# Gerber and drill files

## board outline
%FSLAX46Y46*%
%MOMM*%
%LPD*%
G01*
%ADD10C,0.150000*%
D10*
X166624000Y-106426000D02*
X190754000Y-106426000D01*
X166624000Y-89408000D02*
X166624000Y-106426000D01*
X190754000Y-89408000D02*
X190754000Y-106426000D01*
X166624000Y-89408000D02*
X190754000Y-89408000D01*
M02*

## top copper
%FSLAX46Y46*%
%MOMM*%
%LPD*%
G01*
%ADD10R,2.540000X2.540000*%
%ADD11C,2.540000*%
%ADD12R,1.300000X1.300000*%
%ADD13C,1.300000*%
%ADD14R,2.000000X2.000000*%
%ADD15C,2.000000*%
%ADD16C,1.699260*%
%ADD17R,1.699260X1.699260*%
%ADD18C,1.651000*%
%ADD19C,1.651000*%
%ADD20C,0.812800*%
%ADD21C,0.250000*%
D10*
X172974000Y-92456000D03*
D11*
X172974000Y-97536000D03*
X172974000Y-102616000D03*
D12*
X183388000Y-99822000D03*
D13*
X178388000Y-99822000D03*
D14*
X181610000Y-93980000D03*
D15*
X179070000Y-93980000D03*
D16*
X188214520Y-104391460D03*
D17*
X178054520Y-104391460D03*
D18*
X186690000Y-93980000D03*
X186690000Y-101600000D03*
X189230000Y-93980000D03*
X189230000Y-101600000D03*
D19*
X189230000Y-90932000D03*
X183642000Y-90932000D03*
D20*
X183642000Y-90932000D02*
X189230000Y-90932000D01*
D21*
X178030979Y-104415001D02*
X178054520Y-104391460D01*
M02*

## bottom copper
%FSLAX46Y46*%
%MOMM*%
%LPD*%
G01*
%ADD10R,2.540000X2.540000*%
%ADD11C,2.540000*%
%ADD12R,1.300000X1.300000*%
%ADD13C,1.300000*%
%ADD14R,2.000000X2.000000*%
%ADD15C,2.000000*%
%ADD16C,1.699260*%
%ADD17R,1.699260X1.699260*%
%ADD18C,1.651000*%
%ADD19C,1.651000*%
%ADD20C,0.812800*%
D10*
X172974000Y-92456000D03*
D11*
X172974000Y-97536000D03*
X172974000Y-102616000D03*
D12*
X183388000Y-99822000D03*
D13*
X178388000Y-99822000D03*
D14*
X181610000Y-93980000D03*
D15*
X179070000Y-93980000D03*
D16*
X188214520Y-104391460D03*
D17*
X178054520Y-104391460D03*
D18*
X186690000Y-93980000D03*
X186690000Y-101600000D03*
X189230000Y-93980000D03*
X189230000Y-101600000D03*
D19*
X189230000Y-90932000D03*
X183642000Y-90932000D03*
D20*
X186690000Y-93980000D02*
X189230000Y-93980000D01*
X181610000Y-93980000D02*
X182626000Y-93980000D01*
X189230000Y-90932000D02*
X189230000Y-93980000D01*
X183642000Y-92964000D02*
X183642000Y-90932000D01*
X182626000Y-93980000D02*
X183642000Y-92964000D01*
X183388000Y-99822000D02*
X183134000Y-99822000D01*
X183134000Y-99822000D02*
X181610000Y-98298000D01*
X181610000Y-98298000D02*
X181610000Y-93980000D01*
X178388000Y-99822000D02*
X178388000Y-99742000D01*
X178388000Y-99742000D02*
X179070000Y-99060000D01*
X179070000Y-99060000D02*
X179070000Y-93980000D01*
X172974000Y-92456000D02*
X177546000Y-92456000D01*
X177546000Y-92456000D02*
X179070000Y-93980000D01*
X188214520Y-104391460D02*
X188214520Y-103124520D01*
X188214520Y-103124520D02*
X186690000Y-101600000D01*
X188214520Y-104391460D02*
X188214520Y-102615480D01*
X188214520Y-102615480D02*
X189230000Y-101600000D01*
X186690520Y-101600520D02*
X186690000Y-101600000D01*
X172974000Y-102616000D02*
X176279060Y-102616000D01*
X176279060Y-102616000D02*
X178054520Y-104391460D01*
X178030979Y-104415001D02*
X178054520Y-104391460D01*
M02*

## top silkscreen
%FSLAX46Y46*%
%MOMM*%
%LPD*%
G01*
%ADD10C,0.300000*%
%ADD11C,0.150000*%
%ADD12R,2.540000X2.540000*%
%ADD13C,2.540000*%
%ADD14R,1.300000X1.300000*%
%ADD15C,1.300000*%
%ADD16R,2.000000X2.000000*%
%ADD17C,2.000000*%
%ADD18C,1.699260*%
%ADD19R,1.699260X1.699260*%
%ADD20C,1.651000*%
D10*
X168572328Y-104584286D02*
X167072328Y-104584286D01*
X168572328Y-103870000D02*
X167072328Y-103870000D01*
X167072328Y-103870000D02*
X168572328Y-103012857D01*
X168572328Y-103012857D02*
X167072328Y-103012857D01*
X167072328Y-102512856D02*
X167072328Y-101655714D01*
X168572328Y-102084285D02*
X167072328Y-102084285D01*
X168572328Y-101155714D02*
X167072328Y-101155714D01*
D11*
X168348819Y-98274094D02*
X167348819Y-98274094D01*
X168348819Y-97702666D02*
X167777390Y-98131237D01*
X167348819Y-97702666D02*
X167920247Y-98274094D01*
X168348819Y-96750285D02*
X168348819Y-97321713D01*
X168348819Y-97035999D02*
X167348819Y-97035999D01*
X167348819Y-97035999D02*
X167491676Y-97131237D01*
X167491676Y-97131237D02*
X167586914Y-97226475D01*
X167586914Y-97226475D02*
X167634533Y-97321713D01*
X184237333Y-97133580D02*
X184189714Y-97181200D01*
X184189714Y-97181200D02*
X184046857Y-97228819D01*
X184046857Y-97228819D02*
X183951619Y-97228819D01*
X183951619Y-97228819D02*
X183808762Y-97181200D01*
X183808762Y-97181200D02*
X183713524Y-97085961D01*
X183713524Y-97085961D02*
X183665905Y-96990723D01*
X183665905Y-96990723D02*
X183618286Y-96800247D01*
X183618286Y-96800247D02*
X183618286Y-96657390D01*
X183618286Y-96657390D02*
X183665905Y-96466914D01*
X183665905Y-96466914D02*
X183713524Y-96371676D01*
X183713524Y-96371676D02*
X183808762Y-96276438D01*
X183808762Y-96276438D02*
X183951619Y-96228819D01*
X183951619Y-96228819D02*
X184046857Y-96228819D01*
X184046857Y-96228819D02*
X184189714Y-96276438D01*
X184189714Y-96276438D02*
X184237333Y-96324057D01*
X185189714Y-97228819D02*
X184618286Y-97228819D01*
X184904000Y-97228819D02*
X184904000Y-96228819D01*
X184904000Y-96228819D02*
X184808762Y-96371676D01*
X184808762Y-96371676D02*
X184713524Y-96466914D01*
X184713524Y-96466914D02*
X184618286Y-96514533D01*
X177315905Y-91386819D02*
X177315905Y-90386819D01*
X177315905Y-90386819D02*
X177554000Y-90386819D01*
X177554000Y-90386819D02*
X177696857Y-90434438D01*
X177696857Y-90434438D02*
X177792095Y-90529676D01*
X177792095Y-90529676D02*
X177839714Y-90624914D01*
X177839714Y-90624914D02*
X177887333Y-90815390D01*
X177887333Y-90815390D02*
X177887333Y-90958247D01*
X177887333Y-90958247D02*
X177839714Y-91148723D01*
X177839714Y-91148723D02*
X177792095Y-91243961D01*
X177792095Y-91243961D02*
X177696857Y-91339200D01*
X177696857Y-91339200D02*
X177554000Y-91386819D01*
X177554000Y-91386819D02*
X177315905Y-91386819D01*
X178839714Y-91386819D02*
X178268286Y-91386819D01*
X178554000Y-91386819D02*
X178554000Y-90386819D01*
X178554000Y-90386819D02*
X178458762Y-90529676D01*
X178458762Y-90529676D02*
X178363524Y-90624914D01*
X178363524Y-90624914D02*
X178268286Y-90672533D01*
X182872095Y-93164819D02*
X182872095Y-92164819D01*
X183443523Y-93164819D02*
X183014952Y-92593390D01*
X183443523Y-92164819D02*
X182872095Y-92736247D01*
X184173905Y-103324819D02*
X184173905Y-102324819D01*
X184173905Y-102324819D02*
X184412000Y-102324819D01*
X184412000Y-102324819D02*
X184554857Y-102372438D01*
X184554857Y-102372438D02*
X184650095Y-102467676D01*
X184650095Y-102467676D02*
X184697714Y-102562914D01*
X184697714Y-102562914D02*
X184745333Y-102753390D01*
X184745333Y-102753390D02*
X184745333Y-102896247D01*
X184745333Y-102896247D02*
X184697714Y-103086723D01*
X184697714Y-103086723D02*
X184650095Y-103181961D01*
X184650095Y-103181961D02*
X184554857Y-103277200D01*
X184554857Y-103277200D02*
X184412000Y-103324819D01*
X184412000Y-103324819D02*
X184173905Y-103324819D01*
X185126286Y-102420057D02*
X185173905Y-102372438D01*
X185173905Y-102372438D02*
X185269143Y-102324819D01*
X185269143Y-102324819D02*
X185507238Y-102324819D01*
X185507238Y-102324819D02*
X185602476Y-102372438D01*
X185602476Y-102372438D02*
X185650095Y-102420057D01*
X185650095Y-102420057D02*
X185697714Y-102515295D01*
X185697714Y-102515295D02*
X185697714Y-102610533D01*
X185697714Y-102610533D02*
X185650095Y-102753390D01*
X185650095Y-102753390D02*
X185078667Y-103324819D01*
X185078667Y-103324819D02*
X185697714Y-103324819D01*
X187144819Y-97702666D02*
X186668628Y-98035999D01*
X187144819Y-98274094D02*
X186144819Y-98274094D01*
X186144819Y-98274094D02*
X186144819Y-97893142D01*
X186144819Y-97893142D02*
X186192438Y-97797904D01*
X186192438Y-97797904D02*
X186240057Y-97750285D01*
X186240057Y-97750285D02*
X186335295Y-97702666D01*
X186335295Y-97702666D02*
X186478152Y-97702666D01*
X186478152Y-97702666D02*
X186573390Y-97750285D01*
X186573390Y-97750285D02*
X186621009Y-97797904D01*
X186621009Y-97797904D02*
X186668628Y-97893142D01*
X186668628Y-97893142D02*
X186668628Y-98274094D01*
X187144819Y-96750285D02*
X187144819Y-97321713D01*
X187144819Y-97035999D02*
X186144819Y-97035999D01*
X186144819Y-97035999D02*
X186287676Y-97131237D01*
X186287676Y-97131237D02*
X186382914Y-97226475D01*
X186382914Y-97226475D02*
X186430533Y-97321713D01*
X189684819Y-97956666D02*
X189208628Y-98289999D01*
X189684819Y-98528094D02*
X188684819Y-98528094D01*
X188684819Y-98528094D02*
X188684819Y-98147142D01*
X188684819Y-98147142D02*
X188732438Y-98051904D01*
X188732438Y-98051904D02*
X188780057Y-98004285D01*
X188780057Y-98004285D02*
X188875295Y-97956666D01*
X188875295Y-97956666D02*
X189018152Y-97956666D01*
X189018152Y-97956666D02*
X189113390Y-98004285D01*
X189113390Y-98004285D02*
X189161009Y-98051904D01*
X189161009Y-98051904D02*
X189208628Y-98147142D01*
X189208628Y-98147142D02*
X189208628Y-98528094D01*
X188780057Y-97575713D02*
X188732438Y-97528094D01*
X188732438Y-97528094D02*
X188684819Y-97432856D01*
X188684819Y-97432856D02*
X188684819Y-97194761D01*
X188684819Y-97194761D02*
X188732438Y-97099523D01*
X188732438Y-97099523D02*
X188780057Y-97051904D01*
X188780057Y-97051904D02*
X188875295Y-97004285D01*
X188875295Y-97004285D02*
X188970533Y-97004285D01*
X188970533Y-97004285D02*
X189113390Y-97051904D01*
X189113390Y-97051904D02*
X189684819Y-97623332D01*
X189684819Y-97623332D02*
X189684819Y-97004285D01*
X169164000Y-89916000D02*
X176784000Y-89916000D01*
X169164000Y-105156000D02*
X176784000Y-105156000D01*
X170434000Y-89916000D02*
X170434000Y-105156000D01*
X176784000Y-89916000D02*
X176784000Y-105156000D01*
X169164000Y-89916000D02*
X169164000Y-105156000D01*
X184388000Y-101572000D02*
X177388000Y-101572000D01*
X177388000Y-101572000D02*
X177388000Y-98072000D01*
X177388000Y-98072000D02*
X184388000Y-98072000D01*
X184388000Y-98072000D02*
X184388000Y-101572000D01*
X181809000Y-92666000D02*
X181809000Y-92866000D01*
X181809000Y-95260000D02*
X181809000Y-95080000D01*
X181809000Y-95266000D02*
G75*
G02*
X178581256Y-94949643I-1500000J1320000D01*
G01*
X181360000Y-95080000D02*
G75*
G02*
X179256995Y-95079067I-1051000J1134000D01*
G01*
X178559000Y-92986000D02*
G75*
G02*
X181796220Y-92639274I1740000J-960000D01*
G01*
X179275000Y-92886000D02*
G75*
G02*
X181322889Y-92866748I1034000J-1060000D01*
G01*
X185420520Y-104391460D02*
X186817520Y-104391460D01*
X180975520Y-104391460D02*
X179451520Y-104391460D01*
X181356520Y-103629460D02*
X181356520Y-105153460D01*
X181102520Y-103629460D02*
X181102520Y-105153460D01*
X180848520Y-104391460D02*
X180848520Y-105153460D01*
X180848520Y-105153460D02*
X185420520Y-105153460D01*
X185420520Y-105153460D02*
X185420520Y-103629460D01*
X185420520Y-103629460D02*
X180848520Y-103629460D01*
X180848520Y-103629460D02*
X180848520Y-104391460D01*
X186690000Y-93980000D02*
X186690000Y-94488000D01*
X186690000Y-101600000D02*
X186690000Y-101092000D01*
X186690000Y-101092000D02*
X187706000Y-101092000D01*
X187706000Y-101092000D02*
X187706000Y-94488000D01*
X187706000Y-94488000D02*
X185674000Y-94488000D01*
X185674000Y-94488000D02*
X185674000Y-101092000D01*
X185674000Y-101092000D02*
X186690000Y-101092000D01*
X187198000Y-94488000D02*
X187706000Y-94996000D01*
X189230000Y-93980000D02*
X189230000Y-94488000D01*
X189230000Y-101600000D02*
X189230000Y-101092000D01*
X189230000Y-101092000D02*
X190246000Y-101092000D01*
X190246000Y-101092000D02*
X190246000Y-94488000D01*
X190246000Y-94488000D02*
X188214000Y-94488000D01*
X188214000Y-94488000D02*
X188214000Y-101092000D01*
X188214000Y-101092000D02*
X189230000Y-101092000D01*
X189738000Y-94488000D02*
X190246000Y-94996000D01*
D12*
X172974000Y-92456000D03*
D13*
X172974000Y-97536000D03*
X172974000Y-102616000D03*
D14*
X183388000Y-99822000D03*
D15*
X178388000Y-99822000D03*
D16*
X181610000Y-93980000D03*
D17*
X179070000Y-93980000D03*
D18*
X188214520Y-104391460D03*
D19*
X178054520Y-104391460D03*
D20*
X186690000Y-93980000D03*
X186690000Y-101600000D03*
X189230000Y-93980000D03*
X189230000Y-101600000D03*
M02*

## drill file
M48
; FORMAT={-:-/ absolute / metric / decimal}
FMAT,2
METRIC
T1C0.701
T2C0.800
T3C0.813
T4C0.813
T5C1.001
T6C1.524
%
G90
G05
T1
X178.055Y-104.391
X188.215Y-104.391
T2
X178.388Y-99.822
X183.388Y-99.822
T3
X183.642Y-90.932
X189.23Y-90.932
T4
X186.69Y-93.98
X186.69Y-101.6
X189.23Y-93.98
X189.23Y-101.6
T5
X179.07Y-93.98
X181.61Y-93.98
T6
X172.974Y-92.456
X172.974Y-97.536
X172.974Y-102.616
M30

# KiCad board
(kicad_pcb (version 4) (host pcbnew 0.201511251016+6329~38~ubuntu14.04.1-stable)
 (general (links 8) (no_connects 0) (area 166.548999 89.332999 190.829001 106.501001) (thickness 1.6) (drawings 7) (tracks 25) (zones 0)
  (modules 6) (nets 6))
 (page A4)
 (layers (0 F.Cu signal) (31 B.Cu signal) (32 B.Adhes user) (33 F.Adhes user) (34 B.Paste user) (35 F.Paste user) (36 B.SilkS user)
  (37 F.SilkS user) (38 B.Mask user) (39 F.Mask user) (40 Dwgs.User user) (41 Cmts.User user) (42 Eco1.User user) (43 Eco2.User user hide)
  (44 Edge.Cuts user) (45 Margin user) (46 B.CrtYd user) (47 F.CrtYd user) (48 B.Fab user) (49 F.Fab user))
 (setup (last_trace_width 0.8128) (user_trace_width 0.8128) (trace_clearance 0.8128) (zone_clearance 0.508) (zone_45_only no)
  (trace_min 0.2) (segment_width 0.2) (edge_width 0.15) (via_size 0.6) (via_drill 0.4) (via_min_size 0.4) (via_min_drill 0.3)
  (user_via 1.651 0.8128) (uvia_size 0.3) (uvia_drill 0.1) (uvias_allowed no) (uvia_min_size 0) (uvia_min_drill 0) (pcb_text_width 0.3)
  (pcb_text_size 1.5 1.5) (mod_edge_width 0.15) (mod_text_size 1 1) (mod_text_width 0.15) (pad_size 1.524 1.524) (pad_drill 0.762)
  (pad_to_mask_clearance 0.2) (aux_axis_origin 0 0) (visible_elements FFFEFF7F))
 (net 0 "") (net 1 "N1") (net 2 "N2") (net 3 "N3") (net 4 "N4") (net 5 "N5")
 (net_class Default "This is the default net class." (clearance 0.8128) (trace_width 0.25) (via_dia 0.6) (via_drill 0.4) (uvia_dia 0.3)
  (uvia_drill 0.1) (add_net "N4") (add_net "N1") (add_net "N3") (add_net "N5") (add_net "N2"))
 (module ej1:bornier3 (layer F.Cu) (at 172.974 97.536 270)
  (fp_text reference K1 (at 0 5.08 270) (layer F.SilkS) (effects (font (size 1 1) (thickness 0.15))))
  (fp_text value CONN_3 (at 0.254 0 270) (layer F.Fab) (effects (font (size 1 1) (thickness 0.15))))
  (fp_line (start -7.62 3.81) (end -7.62 -3.81) (layer F.SilkS) (width 0.15))
  (fp_line (start 7.62 3.81) (end 7.62 -3.81) (layer F.SilkS) (width 0.15))
  (fp_line (start -7.62 2.54) (end 7.62 2.54) (layer F.SilkS) (width 0.15))
  (fp_line (start -7.62 -3.81) (end 7.62 -3.81) (layer F.SilkS) (width 0.15))
  (fp_line (start -7.62 3.81) (end 7.62 3.81) (layer F.SilkS) (width 0.15))
  (pad 1 thru_hole rect (at -5.08 0 270) (size 2.54 2.54) (drill 1.524) (layers *.Cu *.Mask F.SilkS) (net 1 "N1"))
  (pad 2 thru_hole circle (at 0 0 270) (size 2.54 2.54) (drill 1.524) (layers *.Cu *.Mask F.SilkS) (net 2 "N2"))
  (pad 3 thru_hole circle (at 5.08 0 270) (size 2.54 2.54) (drill 1.524) (layers *.Cu *.Mask F.SilkS) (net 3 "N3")))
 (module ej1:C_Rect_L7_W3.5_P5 (layer F.Cu) (at 183.388 99.822 180)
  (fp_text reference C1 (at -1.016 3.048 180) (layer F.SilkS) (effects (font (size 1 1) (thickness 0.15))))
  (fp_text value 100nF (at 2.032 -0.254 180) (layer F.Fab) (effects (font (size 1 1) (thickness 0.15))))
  (fp_line (start -1 -1.75) (end 6 -1.75) (layer F.SilkS) (width 0.15))
  (fp_line (start 6 -1.75) (end 6 1.75) (layer F.SilkS) (width 0.15))
  (fp_line (start 6 1.75) (end -1 1.75) (layer F.SilkS) (width 0.15))
  (fp_line (start -1 1.75) (end -1 -1.75) (layer F.SilkS) (width 0.15))
  (pad 1 thru_hole rect (at 0 0 180) (size 1.3 1.3) (drill 0.8) (layers *.Cu *.Mask F.SilkS) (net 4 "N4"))
  (pad 2 thru_hole circle (at 5 0 180) (size 1.3 1.3) (drill 0.8) (layers *.Cu *.Mask F.SilkS) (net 1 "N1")))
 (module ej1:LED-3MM (layer F.Cu) (at 181.61 93.98 180)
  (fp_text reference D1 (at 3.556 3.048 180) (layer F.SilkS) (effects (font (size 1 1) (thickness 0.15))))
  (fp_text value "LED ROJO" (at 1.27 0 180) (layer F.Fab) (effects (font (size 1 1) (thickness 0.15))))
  (fp_line (start -0.199 1.314) (end -0.199 1.114) (layer F.SilkS) (width 0.15))
  (fp_line (start -0.199 -1.28) (end -0.199 -1.1) (layer F.SilkS) (width 0.15))
  (fp_arc (start 1.301 0.034) (end -0.199 -1.286) (angle 108.5) (layer F.SilkS) (width 0.15))
  (fp_arc (start 1.301 0.034) (end 0.25 -1.1) (angle 85.7) (layer F.SilkS) (width 0.15))
  (fp_arc (start 1.311 0.034) (end 3.051 0.994) (angle 110) (layer F.SilkS) (width 0.15))
  (fp_arc (start 1.301 0.034) (end 2.335 1.094) (angle 87.5) (layer F.SilkS) (width 0.15))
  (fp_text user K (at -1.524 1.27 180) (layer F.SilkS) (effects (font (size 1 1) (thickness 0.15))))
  (pad 1 thru_hole rect (at 0 0 270) (size 2 2) (drill 1.00076) (layers *.Cu *.Mask F.SilkS) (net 4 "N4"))
  (pad 2 thru_hole circle (at 2.54 0 180) (size 2 2) (drill 1.00076) (layers *.Cu *.Mask F.SilkS) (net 1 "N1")))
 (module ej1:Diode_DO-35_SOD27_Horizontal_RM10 (layer F.Cu) (at 178.054 104.394)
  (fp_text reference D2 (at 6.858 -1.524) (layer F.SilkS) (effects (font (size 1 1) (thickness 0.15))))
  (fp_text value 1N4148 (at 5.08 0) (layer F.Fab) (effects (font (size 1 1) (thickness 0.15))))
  (fp_line (start 7.36652 -0.00254) (end 8.76352 -0.00254) (layer F.SilkS) (width 0.15))
  (fp_line (start 2.92152 -0.00254) (end 1.39752 -0.00254) (layer F.SilkS) (width 0.15))
  (fp_line (start 3.30252 -0.76454) (end 3.30252 0.75946) (layer F.SilkS) (width 0.15))
  (fp_line (start 3.04852 -0.76454) (end 3.04852 0.75946) (layer F.SilkS) (width 0.15))
  (fp_line (start 2.79452 -0.00254) (end 2.79452 0.75946) (layer F.SilkS) (width 0.15))
  (fp_line (start 2.79452 0.75946) (end 7.36652 0.75946) (layer F.SilkS) (width 0.15))
  (fp_line (start 7.36652 0.75946) (end 7.36652 -0.76454) (layer F.SilkS) (width 0.15))
  (fp_line (start 7.36652 -0.76454) (end 2.79452 -0.76454) (layer F.SilkS) (width 0.15))
  (fp_line (start 2.79452 -0.76454) (end 2.79452 -0.00254) (layer F.SilkS) (width 0.15))
  (pad 2 thru_hole circle (at 10.16052 -0.00254 180) (size 1.69926 1.69926) (drill 0.70104) (layers *.Cu *.Mask F.SilkS) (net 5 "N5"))
  (pad 1 thru_hole rect (at 0.00052 -0.00254 180) (size 1.69926 1.69926) (drill 0.70104) (layers *.Cu *.Mask F.SilkS) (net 3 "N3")))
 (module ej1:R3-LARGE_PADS (layer F.Cu) (at 186.69 97.79 270)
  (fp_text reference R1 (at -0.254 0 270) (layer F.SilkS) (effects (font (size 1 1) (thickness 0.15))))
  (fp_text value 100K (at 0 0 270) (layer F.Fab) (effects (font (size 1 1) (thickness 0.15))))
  (fp_line (start -3.81 0) (end -3.302 0) (layer F.SilkS) (width 0.15))
  (fp_line (start 3.81 0) (end 3.302 0) (layer F.SilkS) (width 0.15))
  (fp_line (start 3.302 0) (end 3.302 -1.016) (layer F.SilkS) (width 0.15))
  (fp_line (start 3.302 -1.016) (end -3.302 -1.016) (layer F.SilkS) (width 0.15))
  (fp_line (start -3.302 -1.016) (end -3.302 1.016) (layer F.SilkS) (width 0.15))
  (fp_line (start -3.302 1.016) (end 3.302 1.016) (layer F.SilkS) (width 0.15))
  (fp_line (start 3.302 1.016) (end 3.302 0) (layer F.SilkS) (width 0.15))
  (fp_line (start -3.302 -0.508) (end -2.794 -1.016) (layer F.SilkS) (width 0.15))
  (pad 1 thru_hole circle (at -3.81 0 270) (size 1.651 1.651) (drill 0.8128) (layers *.Cu *.Mask F.SilkS) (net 4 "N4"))
  (pad 2 thru_hole circle (at 3.81 0 270) (size 1.651 1.651) (drill 0.8128) (layers *.Cu *.Mask F.SilkS) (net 5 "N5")))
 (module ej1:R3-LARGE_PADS (layer F.Cu) (at 189.23 97.79 270)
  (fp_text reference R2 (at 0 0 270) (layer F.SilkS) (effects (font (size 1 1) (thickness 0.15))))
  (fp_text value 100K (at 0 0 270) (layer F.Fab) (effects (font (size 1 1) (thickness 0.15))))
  (fp_line (start -3.81 0) (end -3.302 0) (layer F.SilkS) (width 0.15))
  (fp_line (start 3.81 0) (end 3.302 0) (layer F.SilkS) (width 0.15))
  (fp_line (start 3.302 0) (end 3.302 -1.016) (layer F.SilkS) (width 0.15))
  (fp_line (start 3.302 -1.016) (end -3.302 -1.016) (layer F.SilkS) (width 0.15))
  (fp_line (start -3.302 -1.016) (end -3.302 1.016) (layer F.SilkS) (width 0.15))
  (fp_line (start -3.302 1.016) (end 3.302 1.016) (layer F.SilkS) (width 0.15))
  (fp_line (start 3.302 1.016) (end 3.302 0) (layer F.SilkS) (width 0.15))
  (fp_line (start -3.302 -0.508) (end -2.794 -1.016) (layer F.SilkS) (width 0.15))
  (pad 1 thru_hole circle (at -3.81 0 270) (size 1.651 1.651) (drill 0.8128) (layers *.Cu *.Mask F.SilkS) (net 4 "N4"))
  (pad 2 thru_hole circle (at 3.81 0 270) (size 1.651 1.651) (drill 0.8128) (layers *.Cu *.Mask F.SilkS) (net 5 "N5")))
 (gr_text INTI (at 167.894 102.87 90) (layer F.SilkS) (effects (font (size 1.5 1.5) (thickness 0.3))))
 (gr_line (start 166.624 106.426) (end 190.754 106.426) (angle 90) (layer Edge.Cuts) (width 0.15))
 (gr_line (start 166.624 89.408) (end 166.624 106.426) (angle 90) (layer Edge.Cuts) (width 0.15))
 (gr_line (start 190.754 89.408) (end 190.754 106.426) (angle 90) (layer Edge.Cuts) (width 0.15))
 (gr_line (start 166.624 89.408) (end 190.754 89.408) (angle 90) (layer Edge.Cuts) (width 0.15))
 (segment (start 186.69 93.98) (end 189.23 93.98) (width 0.8128) (layer B.Cu) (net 4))
 (segment (start 181.61 93.98) (end 182.626 93.98) (width 0.8128) (layer B.Cu) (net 4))
 (segment (start 189.23 90.932) (end 189.23 93.98) (width 0.8128) (layer B.Cu) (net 4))
 (via (at 189.23 90.932) (size 1.651) (drill 0.8128) (layers F.Cu B.Cu) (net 4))
 (segment (start 183.642 90.932) (end 189.23 90.932) (width 0.8128) (layer F.Cu) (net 4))
 (via (at 183.642 90.932) (size 1.651) (drill 0.8128) (layers F.Cu B.Cu) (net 4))
 (segment (start 183.642 92.964) (end 183.642 90.932) (width 0.8128) (layer B.Cu) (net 4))
 (segment (start 182.626 93.98) (end 183.642 92.964) (width 0.8128) (layer B.Cu) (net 4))
 (segment (start 183.388 99.822) (end 183.134 99.822) (width 0.8128) (layer B.Cu) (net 4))
 (segment (start 183.134 99.822) (end 181.61 98.298) (width 0.8128) (layer B.Cu) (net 4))
 (segment (start 181.61 98.298) (end 181.61 93.98) (width 0.8128) (layer B.Cu) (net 4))
 (segment (start 178.388 99.822) (end 178.388 99.742) (width 0.8128) (layer B.Cu) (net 1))
 (segment (start 178.388 99.742) (end 179.07 99.06) (width 0.8128) (layer B.Cu) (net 1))
 (segment (start 179.07 99.06) (end 179.07 93.98) (width 0.8128) (layer B.Cu) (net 1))
 (segment (start 172.974 92.456) (end 177.546 92.456) (width 0.8128) (layer B.Cu) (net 1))
 (segment (start 177.546 92.456) (end 179.07 93.98) (width 0.8128) (layer B.Cu) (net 1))
 (segment (start 188.21452 104.39146) (end 188.21452 103.12452) (width 0.8128) (layer B.Cu) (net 5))
 (segment (start 188.21452 103.12452) (end 186.69 101.6) (width 0.8128) (layer B.Cu) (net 5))
 (segment (start 188.21452 104.39146) (end 188.21452 102.61548) (width 0.8128) (layer B.Cu) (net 5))
 (segment (start 188.21452 102.61548) (end 189.23 101.6) (width 0.8128) (layer B.Cu) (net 5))
 (segment (start 186.69052 101.60052) (end 186.69 101.6) (width 0.8128) (layer B.Cu) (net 5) (status 30))
 (segment (start 172.974 102.616) (end 176.27906 102.616) (width 0.8128) (layer B.Cu) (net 3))
 (segment (start 176.27906 102.616) (end 178.05452 104.39146) (width 0.8128) (layer B.Cu) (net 3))
 (segment (start 178.030979 104.415001) (end 178.05452 104.39146) (width 0.8128) (layer B.Cu) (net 3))
 (segment (start 178.030979 104.415001) (end 178.05452 104.39146) (width 0.25) (layer F.Cu) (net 3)))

